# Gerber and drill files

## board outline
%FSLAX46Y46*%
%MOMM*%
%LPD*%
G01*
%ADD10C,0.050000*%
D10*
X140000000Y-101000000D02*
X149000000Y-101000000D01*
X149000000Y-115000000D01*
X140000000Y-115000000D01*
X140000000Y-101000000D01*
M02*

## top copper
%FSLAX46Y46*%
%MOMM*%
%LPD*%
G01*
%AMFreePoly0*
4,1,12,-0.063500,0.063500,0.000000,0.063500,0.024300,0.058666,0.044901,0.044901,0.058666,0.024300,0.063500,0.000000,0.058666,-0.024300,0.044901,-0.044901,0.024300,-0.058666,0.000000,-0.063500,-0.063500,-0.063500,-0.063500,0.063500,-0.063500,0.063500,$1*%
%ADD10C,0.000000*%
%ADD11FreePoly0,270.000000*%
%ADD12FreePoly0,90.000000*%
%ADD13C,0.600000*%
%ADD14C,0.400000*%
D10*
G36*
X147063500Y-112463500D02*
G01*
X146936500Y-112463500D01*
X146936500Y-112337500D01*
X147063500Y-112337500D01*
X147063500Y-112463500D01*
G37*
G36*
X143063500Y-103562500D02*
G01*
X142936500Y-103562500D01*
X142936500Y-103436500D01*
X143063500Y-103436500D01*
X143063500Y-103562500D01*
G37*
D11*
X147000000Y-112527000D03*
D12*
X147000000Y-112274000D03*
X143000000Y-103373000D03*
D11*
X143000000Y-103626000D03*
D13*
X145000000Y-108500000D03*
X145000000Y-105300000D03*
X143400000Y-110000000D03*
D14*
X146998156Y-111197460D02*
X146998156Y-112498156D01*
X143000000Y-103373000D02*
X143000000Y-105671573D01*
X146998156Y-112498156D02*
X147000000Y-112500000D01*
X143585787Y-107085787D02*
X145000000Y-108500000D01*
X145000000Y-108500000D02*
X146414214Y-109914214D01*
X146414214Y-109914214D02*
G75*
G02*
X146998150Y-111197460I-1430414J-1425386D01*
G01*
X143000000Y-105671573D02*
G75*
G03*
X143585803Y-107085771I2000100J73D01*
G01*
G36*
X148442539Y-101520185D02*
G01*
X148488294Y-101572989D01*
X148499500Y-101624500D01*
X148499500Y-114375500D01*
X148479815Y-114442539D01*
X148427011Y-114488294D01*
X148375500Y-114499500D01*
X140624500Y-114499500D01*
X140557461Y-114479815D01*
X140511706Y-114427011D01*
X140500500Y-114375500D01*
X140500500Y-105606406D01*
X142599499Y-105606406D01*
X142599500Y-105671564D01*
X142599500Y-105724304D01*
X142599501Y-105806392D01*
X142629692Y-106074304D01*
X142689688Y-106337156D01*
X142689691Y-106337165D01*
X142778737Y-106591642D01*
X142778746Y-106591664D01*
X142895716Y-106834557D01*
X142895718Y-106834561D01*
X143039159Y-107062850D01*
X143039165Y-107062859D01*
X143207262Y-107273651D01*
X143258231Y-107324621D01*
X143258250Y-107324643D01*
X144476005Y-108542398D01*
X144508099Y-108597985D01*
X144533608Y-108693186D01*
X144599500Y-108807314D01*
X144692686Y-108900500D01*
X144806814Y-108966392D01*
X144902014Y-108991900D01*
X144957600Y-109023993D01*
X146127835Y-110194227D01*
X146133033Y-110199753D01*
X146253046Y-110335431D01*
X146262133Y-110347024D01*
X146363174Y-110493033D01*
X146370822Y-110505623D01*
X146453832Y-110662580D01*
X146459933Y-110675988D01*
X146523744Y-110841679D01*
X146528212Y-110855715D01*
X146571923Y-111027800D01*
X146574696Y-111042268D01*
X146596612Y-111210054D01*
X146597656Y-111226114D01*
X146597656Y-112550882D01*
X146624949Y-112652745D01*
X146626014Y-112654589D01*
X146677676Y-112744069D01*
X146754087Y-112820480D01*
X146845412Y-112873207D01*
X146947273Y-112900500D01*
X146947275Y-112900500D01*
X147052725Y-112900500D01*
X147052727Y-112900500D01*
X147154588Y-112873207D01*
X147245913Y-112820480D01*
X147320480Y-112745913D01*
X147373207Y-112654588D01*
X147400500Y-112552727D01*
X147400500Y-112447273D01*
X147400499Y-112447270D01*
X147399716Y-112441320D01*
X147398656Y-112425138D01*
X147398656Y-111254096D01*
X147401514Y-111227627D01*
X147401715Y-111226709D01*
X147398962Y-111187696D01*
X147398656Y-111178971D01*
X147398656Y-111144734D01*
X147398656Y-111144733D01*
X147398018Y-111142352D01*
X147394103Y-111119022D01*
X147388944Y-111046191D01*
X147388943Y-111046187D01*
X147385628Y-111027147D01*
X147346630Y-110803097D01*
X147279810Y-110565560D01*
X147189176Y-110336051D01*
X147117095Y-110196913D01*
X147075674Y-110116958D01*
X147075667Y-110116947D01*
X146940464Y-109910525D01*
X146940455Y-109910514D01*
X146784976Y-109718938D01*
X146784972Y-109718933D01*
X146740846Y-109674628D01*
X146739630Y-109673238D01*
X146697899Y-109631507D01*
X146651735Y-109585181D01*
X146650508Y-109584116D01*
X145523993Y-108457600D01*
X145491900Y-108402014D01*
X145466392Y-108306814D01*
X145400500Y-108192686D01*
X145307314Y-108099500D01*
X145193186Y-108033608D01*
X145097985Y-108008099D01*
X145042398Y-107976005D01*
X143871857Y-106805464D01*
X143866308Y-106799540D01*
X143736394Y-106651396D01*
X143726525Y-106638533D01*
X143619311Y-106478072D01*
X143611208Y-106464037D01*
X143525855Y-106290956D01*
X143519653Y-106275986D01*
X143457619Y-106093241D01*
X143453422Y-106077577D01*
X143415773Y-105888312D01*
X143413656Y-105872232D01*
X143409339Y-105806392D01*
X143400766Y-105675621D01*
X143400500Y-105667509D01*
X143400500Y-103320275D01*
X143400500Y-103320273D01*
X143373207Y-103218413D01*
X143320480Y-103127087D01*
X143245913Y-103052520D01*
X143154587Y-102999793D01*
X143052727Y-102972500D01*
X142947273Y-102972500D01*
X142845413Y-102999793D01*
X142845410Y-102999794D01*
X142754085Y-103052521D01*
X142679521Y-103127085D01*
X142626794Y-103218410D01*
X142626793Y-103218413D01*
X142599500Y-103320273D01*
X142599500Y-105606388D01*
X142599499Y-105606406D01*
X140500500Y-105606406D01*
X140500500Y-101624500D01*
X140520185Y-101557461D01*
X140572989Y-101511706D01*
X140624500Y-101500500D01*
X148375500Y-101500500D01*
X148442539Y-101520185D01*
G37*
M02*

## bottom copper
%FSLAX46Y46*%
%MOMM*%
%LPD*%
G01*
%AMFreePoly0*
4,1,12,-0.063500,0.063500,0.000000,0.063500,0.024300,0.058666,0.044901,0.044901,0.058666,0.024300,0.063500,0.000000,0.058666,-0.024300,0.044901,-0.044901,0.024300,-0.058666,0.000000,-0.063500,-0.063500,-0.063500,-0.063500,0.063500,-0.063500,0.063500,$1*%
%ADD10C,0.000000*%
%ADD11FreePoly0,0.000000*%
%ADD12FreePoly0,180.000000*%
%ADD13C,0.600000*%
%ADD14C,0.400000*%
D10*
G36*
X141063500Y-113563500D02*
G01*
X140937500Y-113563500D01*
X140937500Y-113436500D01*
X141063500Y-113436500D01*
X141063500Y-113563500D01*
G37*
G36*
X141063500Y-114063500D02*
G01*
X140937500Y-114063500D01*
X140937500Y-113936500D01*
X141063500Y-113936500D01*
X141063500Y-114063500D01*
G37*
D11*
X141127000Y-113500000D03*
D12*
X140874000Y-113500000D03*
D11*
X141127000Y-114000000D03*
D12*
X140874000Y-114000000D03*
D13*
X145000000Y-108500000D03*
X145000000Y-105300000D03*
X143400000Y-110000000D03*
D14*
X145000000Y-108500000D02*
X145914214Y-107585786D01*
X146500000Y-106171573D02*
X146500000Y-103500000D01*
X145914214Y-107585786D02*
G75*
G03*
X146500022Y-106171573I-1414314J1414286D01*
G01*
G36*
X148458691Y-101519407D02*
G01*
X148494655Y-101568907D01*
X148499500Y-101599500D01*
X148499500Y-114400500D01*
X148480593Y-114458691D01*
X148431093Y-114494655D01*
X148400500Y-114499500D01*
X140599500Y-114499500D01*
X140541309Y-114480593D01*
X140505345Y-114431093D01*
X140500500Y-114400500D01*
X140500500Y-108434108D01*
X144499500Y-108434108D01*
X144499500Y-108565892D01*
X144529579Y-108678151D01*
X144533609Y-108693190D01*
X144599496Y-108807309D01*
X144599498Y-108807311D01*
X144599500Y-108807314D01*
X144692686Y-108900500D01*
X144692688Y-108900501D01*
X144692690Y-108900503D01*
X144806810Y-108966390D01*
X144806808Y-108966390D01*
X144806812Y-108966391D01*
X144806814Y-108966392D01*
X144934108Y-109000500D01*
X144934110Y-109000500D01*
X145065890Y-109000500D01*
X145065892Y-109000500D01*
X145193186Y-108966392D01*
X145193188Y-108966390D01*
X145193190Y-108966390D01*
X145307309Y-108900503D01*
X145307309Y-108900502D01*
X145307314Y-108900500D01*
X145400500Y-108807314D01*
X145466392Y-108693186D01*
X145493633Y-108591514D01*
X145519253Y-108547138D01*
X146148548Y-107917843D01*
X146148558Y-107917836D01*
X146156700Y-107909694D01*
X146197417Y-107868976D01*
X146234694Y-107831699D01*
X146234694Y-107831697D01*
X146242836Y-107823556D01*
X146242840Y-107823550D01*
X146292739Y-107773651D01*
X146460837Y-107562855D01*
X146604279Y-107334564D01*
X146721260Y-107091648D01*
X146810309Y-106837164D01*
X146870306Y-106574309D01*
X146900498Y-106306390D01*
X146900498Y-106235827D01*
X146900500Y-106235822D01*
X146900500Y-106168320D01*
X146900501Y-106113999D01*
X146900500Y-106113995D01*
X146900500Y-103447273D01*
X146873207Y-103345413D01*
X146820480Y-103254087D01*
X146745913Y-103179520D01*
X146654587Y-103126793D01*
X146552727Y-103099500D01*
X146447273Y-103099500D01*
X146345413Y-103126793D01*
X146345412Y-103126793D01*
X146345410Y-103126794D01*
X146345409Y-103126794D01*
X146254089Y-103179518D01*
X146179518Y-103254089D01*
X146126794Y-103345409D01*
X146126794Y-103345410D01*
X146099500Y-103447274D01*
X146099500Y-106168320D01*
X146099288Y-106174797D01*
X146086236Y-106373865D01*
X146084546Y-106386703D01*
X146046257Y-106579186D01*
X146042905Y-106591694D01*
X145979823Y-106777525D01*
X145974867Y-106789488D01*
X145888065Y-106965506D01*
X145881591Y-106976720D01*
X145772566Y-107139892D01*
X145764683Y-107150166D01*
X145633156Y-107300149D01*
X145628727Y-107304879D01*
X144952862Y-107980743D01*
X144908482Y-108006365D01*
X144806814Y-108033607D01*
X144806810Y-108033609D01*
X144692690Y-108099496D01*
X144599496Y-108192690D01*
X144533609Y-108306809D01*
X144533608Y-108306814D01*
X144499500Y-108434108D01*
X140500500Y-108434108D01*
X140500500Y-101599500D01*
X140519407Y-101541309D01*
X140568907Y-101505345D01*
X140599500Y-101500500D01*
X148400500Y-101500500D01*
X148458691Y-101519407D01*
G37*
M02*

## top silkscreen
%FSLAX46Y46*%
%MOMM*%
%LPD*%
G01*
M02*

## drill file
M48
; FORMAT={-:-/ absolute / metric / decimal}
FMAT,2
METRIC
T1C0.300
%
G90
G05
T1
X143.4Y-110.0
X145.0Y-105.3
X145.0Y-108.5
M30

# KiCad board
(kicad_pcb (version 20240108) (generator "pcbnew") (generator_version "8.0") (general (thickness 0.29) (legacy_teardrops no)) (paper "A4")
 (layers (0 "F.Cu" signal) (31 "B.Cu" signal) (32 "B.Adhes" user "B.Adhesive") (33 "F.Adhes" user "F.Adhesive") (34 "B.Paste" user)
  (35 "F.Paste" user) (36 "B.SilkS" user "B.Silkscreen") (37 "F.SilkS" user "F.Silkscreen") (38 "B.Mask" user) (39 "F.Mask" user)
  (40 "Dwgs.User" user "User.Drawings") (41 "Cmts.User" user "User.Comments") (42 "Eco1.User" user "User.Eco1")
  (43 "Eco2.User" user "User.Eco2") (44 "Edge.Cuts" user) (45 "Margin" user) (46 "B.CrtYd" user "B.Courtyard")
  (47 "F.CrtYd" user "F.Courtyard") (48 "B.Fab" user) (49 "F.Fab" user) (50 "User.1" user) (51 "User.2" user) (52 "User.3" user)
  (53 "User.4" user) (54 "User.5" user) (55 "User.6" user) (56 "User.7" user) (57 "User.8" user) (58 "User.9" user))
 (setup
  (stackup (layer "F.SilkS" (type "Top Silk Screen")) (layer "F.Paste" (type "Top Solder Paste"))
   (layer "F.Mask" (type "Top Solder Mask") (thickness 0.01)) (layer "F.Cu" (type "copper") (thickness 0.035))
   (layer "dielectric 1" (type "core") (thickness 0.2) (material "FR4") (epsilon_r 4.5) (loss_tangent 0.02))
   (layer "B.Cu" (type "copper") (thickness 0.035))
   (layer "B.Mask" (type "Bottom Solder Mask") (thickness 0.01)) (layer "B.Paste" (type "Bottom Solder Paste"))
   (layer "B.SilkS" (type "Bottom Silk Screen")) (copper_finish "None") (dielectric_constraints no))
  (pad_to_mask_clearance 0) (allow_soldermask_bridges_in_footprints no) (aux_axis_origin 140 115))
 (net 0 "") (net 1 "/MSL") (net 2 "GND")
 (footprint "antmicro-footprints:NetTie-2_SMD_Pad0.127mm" (layer "F.Cu") (at 147 112.4 90)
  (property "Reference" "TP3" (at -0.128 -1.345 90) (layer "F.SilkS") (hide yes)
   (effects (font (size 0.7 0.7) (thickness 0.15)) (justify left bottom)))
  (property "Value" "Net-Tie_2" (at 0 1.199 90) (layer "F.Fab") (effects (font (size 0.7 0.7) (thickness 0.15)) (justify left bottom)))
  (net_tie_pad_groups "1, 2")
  (fp_poly
   (pts (xy -0.0635 -0.0635) (xy 0.0625 -0.0635) (xy 0.0625 0.0635) (xy -0.0635 0.0635)) (stroke (width 0) (type solid)) (fill solid)
   (layer "F.Cu"))
  (pad "1" smd roundrect (at -0.127 0 270) (size 0.127 0.127) (layers "F.Cu") (roundrect_rratio 0.5) (chamfer_ratio 0)
   (chamfer top_left bottom_left) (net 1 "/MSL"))
  (pad "2" smd roundrect (at 0.126 0 90) (size 0.127 0.127) (layers "F.Cu") (roundrect_rratio 0.5) (chamfer_ratio 0)
   (chamfer top_left bottom_left) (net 1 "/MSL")))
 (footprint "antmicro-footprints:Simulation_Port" (layer "F.Cu") (at 147 112.75)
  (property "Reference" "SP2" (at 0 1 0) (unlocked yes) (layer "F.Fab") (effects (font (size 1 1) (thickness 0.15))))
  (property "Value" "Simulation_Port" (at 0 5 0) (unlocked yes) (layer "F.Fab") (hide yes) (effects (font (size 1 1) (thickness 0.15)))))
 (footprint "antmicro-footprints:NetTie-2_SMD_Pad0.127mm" (layer "F.Cu") (at 143 103.5 -90)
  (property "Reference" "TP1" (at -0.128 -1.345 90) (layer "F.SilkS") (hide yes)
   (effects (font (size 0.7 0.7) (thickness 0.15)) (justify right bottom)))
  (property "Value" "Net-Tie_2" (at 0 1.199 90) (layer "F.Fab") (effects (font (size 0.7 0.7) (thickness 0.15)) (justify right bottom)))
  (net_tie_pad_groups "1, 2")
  (fp_poly
   (pts (xy -0.0635 -0.0635) (xy 0.0625 -0.0635) (xy 0.0625 0.0635) (xy -0.0635 0.0635)) (stroke (width 0) (type solid)) (fill solid)
   (layer "F.Cu"))
  (pad "1" smd roundrect (at -0.127 0 90) (size 0.127 0.127) (layers "F.Cu") (roundrect_rratio 0.5) (chamfer_ratio 0)
   (chamfer top_left bottom_left) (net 1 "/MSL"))
  (pad "2" smd roundrect (at 0.126 0 270) (size 0.127 0.127) (layers "F.Cu") (roundrect_rratio 0.5) (chamfer_ratio 0)
   (chamfer top_left bottom_left) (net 1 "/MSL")))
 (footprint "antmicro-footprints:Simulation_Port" (layer "F.Cu") (at 143 103.25 180)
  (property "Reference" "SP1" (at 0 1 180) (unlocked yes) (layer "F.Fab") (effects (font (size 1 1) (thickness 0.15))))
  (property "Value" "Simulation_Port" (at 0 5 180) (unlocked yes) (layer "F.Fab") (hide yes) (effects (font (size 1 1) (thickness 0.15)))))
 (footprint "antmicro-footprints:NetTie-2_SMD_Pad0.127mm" (layer "B.Cu") (at 141 113.5 180)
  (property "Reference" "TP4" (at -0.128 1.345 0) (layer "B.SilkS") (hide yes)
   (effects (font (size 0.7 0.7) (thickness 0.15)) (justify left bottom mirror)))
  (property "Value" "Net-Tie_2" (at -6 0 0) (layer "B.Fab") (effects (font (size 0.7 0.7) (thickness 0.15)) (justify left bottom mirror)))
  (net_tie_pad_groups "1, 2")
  (fp_poly
   (pts (xy -0.0635 0.0635) (xy 0.0625 0.0635) (xy 0.0625 -0.0635) (xy -0.0635 -0.0635)) (stroke (width 0) (type solid)) (fill solid)
   (layer "B.Cu"))
  (pad "1" smd roundrect (at -0.127 0) (size 0.127 0.127) (layers "B.Cu") (roundrect_rratio 0.5) (chamfer_ratio 0)
   (chamfer top_left bottom_left) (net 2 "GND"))
  (pad "2" smd roundrect (at 0.126 0 180) (size 0.127 0.127) (layers "B.Cu") (roundrect_rratio 0.5) (chamfer_ratio 0)
   (chamfer top_left bottom_left) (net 2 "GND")))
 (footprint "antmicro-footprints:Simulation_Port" (layer "B.Cu") (at 146.5 103.25)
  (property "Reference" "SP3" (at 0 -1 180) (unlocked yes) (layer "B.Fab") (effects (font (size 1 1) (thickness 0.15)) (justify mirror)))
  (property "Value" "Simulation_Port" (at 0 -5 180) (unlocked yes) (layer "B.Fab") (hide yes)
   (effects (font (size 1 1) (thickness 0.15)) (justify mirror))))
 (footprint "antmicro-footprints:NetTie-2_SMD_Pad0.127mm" (layer "B.Cu") (at 141 114 180)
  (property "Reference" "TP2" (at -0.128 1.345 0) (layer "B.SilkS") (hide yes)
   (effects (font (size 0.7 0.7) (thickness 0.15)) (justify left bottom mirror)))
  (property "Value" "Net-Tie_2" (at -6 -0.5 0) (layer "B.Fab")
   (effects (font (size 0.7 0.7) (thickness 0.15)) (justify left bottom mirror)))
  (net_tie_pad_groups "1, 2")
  (fp_poly
   (pts (xy -0.0635 0.0635) (xy 0.0625 0.0635) (xy 0.0625 -0.0635) (xy -0.0635 -0.0635)) (stroke (width 0) (type solid)) (fill solid)
   (layer "B.Cu"))
  (pad "1" smd roundrect (at -0.127 0) (size 0.127 0.127) (layers "B.Cu") (roundrect_rratio 0.5) (chamfer_ratio 0)
   (chamfer top_left bottom_left) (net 2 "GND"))
  (pad "2" smd roundrect (at 0.126 0 180) (size 0.127 0.127) (layers "B.Cu") (roundrect_rratio 0.5) (chamfer_ratio 0)
   (chamfer top_left bottom_left) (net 2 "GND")))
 (gr_rect (start 140 101) (end 149 115) (stroke (width 0.05) (type solid)) (fill none) (layer "Edge.Cuts"))
 (segment (start 146.998156 111.19746) (end 146.998156 112.498156) (width 0.4) (layer "F.Cu") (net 1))
 (segment (start 143 103.373) (end 143 105.671573) (width 0.4) (layer "F.Cu") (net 1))
 (segment (start 146.998156 112.498156) (end 147 112.5) (width 0.4) (layer "F.Cu") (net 1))
 (segment (start 143.585787 107.085787) (end 145 108.5) (width 0.4) (layer "F.Cu") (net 1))
 (segment (start 145 108.5) (end 146.414214 109.914214) (width 0.4) (layer "F.Cu") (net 1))
 (via (at 145 108.5) (size 0.6) (drill 0.3) (layers "F.Cu" "B.Cu") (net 1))
 (arc (start 146.414214 109.914214) (mid 146.82172 110.503015) (end 146.998156 111.19746) (width 0.4) (layer "F.Cu") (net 1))
 (arc (start 143 105.671573) (mid 143.15225 106.436939) (end 143.585787 107.085787) (width 0.4) (layer "F.Cu") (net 1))
 (segment (start 145 108.5) (end 145.914214 107.585786) (width 0.4) (layer "B.Cu") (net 1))
 (segment (start 146.5 106.171573) (end 146.5 103.5) (width 0.4) (layer "B.Cu") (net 1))
 (arc (start 145.914214 107.585786) (mid 146.34775 106.936938) (end 146.5 106.171573) (width 0.4) (layer "B.Cu") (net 1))
 (via (at 145 105.3) (size 0.6) (drill 0.3) (layers "F.Cu" "B.Cu") (free yes) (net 2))
 (via (at 143.4 110) (size 0.6) (drill 0.3) (layers "F.Cu" "B.Cu") (free yes) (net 2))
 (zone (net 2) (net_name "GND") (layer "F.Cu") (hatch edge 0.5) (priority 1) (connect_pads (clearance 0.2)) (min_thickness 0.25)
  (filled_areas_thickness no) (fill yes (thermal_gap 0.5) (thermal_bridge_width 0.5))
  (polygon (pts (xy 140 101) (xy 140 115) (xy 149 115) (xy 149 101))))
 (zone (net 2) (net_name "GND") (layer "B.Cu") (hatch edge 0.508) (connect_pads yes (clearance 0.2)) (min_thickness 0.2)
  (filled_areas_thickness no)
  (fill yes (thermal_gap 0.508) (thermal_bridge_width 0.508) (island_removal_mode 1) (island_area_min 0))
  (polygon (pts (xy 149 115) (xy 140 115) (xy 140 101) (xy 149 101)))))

